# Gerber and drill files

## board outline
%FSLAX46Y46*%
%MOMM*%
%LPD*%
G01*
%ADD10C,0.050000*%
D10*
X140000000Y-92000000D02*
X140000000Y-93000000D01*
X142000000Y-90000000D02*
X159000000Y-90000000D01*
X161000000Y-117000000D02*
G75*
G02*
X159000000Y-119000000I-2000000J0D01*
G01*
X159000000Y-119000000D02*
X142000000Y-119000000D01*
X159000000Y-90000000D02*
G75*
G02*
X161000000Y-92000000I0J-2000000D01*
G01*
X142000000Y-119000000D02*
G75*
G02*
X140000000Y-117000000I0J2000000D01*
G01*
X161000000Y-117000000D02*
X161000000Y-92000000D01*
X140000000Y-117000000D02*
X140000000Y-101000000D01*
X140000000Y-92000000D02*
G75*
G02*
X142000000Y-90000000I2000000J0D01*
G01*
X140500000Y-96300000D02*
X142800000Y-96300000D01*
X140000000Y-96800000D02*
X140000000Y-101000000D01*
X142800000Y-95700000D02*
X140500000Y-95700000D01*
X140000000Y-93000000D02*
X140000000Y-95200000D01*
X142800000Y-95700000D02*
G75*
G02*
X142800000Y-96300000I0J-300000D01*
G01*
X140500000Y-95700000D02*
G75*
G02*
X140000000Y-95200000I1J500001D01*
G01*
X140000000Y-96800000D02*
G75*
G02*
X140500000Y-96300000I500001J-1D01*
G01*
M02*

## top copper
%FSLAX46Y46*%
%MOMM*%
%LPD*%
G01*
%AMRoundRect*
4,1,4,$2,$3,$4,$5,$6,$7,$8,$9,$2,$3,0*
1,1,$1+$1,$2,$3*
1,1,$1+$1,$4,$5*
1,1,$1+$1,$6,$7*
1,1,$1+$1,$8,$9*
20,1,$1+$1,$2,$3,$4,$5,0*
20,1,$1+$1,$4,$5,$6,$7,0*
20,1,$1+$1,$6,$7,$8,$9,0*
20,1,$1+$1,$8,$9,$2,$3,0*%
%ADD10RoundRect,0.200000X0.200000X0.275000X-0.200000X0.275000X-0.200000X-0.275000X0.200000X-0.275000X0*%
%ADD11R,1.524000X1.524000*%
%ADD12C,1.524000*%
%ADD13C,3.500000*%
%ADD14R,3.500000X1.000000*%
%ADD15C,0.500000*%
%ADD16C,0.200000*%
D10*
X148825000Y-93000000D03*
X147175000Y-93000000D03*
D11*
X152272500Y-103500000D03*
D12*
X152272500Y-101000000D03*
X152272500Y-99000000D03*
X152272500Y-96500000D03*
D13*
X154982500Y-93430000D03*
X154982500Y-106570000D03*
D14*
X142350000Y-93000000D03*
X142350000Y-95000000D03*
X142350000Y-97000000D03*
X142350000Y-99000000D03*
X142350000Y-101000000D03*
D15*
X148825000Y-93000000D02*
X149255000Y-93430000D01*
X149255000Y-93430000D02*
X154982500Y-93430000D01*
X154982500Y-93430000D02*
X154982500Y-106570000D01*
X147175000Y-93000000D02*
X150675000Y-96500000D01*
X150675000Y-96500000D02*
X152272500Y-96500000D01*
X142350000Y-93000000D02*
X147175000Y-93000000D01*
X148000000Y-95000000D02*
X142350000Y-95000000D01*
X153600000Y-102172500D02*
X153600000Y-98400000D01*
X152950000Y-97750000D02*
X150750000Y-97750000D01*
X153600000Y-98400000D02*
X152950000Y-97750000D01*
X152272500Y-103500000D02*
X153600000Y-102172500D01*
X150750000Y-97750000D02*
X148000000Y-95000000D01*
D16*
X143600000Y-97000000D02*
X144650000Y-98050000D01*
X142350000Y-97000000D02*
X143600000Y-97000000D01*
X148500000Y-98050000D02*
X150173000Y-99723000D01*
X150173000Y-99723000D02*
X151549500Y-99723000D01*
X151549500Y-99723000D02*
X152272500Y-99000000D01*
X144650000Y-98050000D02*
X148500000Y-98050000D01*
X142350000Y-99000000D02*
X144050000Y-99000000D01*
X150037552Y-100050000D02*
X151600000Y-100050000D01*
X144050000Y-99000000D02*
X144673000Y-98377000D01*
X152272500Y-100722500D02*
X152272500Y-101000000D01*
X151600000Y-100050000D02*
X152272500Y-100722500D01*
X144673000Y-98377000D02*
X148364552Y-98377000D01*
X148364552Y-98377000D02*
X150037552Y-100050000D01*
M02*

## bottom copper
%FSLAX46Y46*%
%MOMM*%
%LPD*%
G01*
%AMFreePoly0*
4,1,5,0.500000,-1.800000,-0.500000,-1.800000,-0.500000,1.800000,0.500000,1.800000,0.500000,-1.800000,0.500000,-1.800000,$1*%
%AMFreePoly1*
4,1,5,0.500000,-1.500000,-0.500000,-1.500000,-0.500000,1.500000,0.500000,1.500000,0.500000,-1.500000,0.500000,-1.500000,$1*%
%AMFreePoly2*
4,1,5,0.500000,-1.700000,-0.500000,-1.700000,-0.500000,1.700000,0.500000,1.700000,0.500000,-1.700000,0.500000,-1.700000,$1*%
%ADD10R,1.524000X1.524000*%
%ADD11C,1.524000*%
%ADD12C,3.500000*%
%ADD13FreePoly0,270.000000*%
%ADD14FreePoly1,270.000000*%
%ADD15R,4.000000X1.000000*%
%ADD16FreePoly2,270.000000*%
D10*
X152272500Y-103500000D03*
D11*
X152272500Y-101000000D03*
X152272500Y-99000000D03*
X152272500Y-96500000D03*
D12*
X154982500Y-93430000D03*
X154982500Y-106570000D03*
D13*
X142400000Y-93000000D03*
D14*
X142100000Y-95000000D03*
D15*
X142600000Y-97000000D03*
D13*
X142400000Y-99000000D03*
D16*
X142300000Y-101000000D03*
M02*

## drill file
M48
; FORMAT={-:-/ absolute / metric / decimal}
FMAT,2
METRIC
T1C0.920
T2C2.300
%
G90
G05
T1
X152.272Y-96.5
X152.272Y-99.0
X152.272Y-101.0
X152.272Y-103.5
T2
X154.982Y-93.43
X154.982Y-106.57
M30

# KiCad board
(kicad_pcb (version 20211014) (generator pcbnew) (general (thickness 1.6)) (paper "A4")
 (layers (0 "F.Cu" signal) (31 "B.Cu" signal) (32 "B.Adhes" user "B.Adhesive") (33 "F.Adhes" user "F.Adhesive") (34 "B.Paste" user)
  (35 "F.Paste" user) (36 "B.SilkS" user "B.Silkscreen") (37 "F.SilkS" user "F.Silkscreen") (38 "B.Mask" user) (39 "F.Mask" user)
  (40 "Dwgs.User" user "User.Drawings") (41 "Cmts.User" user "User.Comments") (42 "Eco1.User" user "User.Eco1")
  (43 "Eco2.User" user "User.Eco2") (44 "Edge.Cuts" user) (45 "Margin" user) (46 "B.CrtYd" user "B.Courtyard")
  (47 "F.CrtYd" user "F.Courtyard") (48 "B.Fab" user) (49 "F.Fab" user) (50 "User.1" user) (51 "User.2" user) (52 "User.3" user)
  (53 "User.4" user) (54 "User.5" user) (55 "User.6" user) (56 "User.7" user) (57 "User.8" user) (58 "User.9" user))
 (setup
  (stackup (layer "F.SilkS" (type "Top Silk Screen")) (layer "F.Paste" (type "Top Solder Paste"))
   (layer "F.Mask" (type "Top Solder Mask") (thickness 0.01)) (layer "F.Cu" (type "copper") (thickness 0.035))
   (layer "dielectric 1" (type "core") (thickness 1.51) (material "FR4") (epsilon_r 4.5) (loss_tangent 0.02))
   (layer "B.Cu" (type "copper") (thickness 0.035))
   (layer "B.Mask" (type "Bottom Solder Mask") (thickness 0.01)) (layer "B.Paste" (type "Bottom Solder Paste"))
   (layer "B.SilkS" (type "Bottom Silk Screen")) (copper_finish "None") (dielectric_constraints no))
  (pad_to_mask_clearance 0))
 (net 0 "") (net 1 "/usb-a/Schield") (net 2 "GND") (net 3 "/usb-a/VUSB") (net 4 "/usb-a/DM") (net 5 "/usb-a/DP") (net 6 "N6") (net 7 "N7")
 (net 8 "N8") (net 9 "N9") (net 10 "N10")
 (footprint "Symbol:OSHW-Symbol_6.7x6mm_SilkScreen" (layer "F.Cu") (at 146.5 108.4)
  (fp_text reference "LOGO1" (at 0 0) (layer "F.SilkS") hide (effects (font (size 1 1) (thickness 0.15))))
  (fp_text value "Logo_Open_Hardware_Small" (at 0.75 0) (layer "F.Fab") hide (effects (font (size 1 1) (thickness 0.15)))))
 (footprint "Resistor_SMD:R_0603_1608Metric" (layer "F.Cu") (at 148 93 180)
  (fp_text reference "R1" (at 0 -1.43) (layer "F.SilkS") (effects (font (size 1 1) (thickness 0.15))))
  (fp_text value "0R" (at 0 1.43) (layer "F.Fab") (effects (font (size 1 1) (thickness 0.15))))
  (pad "1" smd roundrect (at -0.825 0 180) (size 0.8 0.95) (layers "F.Cu" "F.Paste" "F.Mask") (roundrect_rratio 0.25)
   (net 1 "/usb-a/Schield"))
  (pad "2" smd roundrect (at 0.825 0 180) (size 0.8 0.95) (layers "F.Cu" "F.Paste" "F.Mask") (roundrect_rratio 0.25) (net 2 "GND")))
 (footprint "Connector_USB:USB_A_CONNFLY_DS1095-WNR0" (layer "F.Cu") (at 152.2725 103.5 90)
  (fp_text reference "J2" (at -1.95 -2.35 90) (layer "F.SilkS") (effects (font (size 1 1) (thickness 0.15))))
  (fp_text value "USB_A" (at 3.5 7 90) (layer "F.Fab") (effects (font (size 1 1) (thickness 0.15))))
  (pad "1" thru_hole rect (at 0 0 90) (size 1.524 1.524) (drill 0.92) (layers *.Cu *.Mask) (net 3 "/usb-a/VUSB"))
  (pad "2" thru_hole circle (at 2.5 0 90) (size 1.524 1.524) (drill 0.92) (layers *.Cu *.Mask) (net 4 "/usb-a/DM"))
  (pad "3" thru_hole circle (at 4.5 0 90) (size 1.524 1.524) (drill 0.92) (layers *.Cu *.Mask) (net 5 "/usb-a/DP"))
  (pad "4" thru_hole circle (at 7 0 90) (size 1.524 1.524) (drill 0.92) (layers *.Cu *.Mask) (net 2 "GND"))
  (pad "5" thru_hole circle (at 10.07 2.71 90) (size 3.5 3.5) (drill 2.3) (layers *.Cu *.Mask) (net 1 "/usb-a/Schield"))
  (pad "5" thru_hole circle (at -3.07 2.71 90) (size 3.5 3.5) (drill 2.3) (layers *.Cu *.Mask) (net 1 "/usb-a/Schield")))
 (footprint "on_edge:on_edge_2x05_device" (layer "F.Cu") (at 140 97 -90)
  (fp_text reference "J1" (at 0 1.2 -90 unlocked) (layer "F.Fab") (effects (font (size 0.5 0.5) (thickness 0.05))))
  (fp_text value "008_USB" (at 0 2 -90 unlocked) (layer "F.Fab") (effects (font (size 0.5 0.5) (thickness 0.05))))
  (fp_line (start -0.7 -0.5) (end -0.7 -2.8) (layer "Edge.Cuts") (width 0.05))
  (fp_line (start -0.2 0) (end 4 0) (layer "Edge.Cuts") (width 0.05))
  (fp_line (start -1.3 -2.8) (end -1.3 -0.5) (layer "Edge.Cuts") (width 0.05))
  (fp_line (start -4 0) (end -1.8 0) (layer "Edge.Cuts") (width 0.05))
  (fp_arc (start -1.3 -2.8) (mid -1 -3.1) (end -0.7 -2.8) (layer "Edge.Cuts") (width 0.05))
  (fp_arc (start -1.3 -0.5) (mid -1.446447 -0.146447) (end -1.8 0) (layer "Edge.Cuts") (width 0.05))
  (fp_arc (start -0.2 0) (mid -0.553553 -0.146447) (end -0.7 -0.5) (layer "Edge.Cuts") (width 0.05))
  (pad "1" smd rect (at -4 -2.35 90) (size 1 3.5) (layers "F.Cu" "F.Mask") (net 2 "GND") (zone_connect 0))
  (pad "2" smd rect (at -2 -2.35 270) (size 1 3.5) (layers "F.Cu" "F.Mask") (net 3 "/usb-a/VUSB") (zone_connect 0))
  (pad "3" smd rect (at 0 -2.35 270) (size 1 3.5) (layers "F.Cu" "F.Mask") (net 5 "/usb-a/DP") (zone_connect 0))
  (pad "4" smd rect (at 2 -2.35 90) (size 1 3.5) (layers "F.Cu" "F.Mask") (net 4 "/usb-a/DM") (zone_connect 0))
  (pad "5" smd rect (at 4 -2.35 90) (size 1 3.5) (layers "F.Cu" "F.Mask") (zone_connect 0))
  (pad "6" smd custom (at -4 -2.4 270) (size 1 3.6) (layers "B.Cu" "B.Mask") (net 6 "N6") (zone_connect 0)
   (options (clearance outline) (anchor rect)) (primitives))
  (pad "7" smd custom (at -2 -2.1 270) (size 1 3) (layers "B.Cu" "B.Mask") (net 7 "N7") (zone_connect 0)
   (options (clearance outline) (anchor rect)) (primitives))
  (pad "8" smd rect (at 0 -2.6 270) (size 1 4) (layers "B.Cu" "B.Mask") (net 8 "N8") (zone_connect 0))
  (pad "9" smd custom (at 2 -2.4 270) (size 1 3.6) (layers "B.Cu" "B.Mask") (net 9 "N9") (zone_connect 0)
   (options (clearance outline) (anchor rect)) (primitives))
  (pad "10" smd custom (at 4 -2.3 270) (size 1 3.4) (layers "B.Cu" "B.Mask") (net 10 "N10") (zone_connect 0)
   (options (clearance outline) (anchor rect)) (primitives))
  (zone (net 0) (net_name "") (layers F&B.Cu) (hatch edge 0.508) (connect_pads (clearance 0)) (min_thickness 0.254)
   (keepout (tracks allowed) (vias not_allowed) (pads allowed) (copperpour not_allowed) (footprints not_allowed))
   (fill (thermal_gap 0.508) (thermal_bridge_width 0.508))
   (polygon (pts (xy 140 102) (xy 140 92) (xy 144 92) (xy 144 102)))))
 (gr_line (start 140 92) (end 140 93) (layer "Edge.Cuts") (width 0.05))
 (gr_line (start 142 90) (end 159 90) (layer "Edge.Cuts") (width 0.05))
 (gr_arc (start 161 117) (mid 160.414214 118.414214) (end 159 119) (layer "Edge.Cuts") (width 0.05))
 (gr_line (start 159 119) (end 142 119) (layer "Edge.Cuts") (width 0.05))
 (gr_arc (start 159 90) (mid 160.414214 90.585786) (end 161 92) (layer "Edge.Cuts") (width 0.05))
 (gr_arc (start 142 119) (mid 140.585786 118.414214) (end 140 117) (layer "Edge.Cuts") (width 0.05))
 (gr_line (start 161 117) (end 161 92) (layer "Edge.Cuts") (width 0.05))
 (gr_line (start 140 117) (end 140 101) (layer "Edge.Cuts") (width 0.05))
 (gr_arc (start 140 92) (mid 140.585786 90.585786) (end 142 90) (layer "Edge.Cuts") (width 0.05))
 (segment (start 148.825 93) (end 149.255 93.43) (width 0.5) (layer "F.Cu") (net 1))
 (segment (start 149.255 93.43) (end 154.9825 93.43) (width 0.5) (layer "F.Cu") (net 1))
 (segment (start 154.9825 93.43) (end 154.9825 106.57) (width 0.5) (layer "F.Cu") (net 1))
 (segment (start 147.175 93) (end 150.675 96.5) (width 0.5) (layer "F.Cu") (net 2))
 (segment (start 150.675 96.5) (end 152.2725 96.5) (width 0.5) (layer "F.Cu") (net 2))
 (segment (start 142.35 93) (end 147.175 93) (width 0.5) (layer "F.Cu") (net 2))
 (segment (start 148 95) (end 142.35 95) (width 0.5) (layer "F.Cu") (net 3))
 (segment (start 153.6 102.1725) (end 153.6 98.4) (width 0.5) (layer "F.Cu") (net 3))
 (segment (start 152.95 97.75) (end 150.75 97.75) (width 0.5) (layer "F.Cu") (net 3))
 (segment (start 153.6 98.4) (end 152.95 97.75) (width 0.5) (layer "F.Cu") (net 3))
 (segment (start 152.2725 103.5) (end 153.6 102.1725) (width 0.5) (layer "F.Cu") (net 3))
 (segment (start 150.75 97.75) (end 148 95) (width 0.5) (layer "F.Cu") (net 3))
 (segment (start 143.6 97) (end 144.65 98.05) (width 0.2) (layer "F.Cu") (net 5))
 (segment (start 142.35 97) (end 143.6 97) (width 0.2) (layer "F.Cu") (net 5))
 (segment (start 148.5 98.05) (end 150.173 99.723) (width 0.2) (layer "F.Cu") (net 5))
 (segment (start 150.173 99.723) (end 151.5495 99.723) (width 0.2) (layer "F.Cu") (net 5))
 (segment (start 151.5495 99.723) (end 152.2725 99) (width 0.2) (layer "F.Cu") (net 5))
 (segment (start 144.65 98.05) (end 148.5 98.05) (width 0.2) (layer "F.Cu") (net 5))
 (segment (start 142.35 99) (end 144.05 99) (width 0.2) (layer "F.Cu") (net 4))
 (segment (start 150.037552 100.05) (end 151.6 100.05) (width 0.2) (layer "F.Cu") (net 4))
 (segment (start 144.05 99) (end 144.673 98.377) (width 0.2) (layer "F.Cu") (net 4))
 (segment (start 152.2725 100.7225) (end 152.2725 101) (width 0.2) (layer "F.Cu") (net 4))
 (segment (start 151.6 100.05) (end 152.2725 100.7225) (width 0.2) (layer "F.Cu") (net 4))
 (segment (start 144.673 98.377) (end 148.364552 98.377) (width 0.2) (layer "F.Cu") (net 4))
 (segment (start 148.364552 98.377) (end 150.037552 100.05) (width 0.2) (layer "F.Cu") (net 4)))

